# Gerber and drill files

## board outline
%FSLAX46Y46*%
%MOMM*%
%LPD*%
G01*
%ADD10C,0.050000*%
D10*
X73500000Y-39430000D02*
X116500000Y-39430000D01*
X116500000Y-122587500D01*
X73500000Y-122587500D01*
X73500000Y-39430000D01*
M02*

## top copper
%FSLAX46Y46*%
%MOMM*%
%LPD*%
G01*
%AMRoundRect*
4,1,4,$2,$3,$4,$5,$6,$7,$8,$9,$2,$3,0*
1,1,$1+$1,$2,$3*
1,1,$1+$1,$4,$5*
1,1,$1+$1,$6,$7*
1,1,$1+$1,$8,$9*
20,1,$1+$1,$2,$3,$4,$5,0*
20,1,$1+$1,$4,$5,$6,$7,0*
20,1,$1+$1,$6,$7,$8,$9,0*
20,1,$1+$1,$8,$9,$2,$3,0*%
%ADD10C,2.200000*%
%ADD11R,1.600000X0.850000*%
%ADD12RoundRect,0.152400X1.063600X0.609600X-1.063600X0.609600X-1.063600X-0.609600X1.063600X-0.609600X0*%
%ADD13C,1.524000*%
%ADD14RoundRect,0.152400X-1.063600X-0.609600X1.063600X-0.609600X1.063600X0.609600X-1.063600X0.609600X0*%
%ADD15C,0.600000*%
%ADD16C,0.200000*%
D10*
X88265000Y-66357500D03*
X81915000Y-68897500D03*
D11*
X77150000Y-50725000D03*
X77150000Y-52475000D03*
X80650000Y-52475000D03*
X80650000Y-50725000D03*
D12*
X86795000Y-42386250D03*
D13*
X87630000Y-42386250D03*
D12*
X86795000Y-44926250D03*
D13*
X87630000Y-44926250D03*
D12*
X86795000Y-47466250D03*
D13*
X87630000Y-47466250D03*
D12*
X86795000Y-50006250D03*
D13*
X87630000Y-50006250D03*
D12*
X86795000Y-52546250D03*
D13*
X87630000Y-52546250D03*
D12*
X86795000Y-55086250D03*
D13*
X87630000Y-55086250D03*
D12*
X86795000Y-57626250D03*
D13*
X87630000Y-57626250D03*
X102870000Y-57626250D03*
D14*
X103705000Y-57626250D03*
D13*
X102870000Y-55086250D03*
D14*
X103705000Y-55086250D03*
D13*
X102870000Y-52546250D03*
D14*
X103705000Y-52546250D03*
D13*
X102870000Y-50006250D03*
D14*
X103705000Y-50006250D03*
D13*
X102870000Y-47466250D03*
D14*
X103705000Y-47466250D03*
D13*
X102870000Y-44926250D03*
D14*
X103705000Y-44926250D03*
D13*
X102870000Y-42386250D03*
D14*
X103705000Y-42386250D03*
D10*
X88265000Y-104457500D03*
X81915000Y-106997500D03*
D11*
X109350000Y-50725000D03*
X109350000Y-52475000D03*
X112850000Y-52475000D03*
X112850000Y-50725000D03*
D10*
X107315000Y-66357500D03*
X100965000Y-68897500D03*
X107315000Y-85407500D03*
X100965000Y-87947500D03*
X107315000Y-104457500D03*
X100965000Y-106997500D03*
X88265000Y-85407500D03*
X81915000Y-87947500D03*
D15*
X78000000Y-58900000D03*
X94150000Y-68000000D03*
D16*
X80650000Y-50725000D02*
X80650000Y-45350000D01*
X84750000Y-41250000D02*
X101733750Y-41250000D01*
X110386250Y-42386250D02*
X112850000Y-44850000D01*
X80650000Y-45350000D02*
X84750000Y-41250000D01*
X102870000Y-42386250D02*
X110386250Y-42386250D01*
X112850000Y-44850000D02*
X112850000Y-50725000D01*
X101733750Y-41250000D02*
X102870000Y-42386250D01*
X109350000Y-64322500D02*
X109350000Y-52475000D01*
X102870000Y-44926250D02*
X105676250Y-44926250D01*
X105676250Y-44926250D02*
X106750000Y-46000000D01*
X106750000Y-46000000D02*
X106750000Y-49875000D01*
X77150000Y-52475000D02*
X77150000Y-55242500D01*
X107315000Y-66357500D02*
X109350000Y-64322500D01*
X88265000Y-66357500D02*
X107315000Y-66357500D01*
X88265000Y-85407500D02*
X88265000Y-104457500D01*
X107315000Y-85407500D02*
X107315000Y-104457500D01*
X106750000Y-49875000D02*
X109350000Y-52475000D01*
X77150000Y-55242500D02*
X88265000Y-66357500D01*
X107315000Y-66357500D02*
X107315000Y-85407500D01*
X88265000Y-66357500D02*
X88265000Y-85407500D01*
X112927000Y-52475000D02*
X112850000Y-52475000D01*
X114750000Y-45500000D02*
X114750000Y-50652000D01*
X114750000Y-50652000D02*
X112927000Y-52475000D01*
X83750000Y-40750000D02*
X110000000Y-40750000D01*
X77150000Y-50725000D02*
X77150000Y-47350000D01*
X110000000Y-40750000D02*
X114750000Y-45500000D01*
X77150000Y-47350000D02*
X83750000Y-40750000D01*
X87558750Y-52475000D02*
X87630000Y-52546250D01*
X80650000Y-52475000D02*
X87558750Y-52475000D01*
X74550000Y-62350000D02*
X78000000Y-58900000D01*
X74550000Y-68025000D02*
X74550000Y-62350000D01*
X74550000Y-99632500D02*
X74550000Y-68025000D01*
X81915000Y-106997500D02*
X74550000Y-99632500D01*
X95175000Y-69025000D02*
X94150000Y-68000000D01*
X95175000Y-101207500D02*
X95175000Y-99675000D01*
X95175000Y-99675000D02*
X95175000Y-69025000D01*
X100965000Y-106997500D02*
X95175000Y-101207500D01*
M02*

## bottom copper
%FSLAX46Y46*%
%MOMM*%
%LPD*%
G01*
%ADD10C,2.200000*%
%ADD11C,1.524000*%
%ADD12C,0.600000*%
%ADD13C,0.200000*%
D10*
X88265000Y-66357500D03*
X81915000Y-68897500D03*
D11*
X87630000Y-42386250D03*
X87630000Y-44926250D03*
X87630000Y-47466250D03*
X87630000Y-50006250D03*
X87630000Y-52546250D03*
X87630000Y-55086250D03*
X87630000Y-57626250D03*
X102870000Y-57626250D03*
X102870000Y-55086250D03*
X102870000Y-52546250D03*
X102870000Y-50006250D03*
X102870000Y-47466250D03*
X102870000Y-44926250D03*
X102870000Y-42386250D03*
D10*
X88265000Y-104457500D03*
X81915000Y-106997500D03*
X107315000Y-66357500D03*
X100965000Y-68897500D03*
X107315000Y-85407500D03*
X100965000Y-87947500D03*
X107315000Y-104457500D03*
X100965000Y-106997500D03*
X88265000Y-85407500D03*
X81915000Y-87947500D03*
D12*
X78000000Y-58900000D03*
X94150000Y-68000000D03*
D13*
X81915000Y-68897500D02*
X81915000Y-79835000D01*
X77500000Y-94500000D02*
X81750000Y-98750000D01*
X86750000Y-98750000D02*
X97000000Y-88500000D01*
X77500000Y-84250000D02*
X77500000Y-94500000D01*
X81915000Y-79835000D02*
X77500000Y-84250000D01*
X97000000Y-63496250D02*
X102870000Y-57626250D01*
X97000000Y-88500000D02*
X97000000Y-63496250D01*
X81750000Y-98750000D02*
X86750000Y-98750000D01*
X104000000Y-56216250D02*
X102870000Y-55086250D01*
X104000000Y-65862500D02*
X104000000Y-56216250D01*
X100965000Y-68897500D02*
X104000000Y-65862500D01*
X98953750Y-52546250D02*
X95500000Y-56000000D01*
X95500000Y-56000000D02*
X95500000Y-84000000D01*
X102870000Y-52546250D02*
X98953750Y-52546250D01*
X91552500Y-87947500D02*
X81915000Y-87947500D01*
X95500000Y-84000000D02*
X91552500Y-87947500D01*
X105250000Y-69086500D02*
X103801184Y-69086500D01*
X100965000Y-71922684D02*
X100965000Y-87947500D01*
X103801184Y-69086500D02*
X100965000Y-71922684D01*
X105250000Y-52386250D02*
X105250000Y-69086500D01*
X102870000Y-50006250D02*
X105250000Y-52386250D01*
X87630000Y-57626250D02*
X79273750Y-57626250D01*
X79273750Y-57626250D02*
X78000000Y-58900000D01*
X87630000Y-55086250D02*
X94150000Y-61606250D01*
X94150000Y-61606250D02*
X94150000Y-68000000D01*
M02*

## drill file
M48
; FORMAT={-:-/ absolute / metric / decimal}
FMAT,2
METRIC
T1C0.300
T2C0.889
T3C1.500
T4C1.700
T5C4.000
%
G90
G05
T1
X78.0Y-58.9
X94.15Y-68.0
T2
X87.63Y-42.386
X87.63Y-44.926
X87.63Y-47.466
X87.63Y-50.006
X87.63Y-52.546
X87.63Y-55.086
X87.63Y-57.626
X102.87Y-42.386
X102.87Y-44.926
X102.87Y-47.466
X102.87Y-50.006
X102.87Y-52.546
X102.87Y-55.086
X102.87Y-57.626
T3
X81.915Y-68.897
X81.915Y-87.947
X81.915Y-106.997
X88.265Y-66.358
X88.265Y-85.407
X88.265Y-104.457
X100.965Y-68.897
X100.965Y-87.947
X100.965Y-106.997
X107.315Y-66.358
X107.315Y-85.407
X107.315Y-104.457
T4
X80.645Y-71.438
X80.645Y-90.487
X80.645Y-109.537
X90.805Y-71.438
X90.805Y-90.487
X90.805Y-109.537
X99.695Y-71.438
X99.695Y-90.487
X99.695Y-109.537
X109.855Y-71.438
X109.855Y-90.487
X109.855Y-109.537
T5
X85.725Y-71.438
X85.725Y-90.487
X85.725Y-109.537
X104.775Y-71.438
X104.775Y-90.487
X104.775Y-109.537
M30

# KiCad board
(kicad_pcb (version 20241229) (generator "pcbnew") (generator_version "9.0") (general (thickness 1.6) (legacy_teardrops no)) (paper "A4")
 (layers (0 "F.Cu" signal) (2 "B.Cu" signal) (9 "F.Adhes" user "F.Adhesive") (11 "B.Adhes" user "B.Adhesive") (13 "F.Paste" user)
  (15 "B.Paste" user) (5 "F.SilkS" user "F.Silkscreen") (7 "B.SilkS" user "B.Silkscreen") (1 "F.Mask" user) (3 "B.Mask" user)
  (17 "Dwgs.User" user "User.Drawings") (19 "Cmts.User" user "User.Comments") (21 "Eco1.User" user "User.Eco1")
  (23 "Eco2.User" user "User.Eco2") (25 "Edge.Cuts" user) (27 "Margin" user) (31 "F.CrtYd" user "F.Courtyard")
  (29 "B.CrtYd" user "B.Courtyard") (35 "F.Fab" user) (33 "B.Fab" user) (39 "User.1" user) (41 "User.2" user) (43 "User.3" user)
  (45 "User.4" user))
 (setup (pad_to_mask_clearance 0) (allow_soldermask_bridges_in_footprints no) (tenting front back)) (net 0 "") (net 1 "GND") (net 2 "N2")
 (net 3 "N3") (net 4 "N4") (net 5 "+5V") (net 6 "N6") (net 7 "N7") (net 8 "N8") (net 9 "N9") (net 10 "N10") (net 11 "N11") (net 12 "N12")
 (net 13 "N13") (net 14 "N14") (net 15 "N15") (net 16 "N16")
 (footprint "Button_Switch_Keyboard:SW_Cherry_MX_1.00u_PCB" (layer "F.Cu") (at 88.265 66.3575)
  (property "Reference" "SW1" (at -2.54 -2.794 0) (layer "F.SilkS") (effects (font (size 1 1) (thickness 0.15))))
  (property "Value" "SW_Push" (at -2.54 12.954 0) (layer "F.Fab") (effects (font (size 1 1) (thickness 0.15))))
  (pad "" np_thru_hole circle (at -7.62 5.08) (size 1.7 1.7) (drill 1.7) (layers "*.Cu" "*.Mask"))
  (pad "" np_thru_hole circle (at -2.54 5.08) (size 4 4) (drill 4) (layers "*.Cu" "*.Mask"))
  (pad "" np_thru_hole circle (at 2.54 5.08) (size 1.7 1.7) (drill 1.7) (layers "*.Cu" "*.Mask"))
  (pad "1" thru_hole circle (at 0 0) (size 2.2 2.2) (drill 1.5) (layers "*.Cu" "*.Mask") (remove_unused_layers no) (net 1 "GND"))
  (pad "2" thru_hole circle (at -6.35 2.54) (size 2.2 2.2) (drill 1.5) (layers "*.Cu" "*.Mask") (remove_unused_layers no) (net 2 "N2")))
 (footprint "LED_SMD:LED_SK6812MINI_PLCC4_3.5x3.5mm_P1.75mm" (layer "F.Cu") (at 78.9 51.6)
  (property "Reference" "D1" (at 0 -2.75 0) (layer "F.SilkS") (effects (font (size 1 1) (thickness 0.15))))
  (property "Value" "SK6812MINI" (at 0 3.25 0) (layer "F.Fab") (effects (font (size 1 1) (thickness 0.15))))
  (pad "1" smd rect (at -1.75 -0.875) (size 1.6 0.85) (layers "F.Cu" "F.Mask" "F.Paste") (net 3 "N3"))
  (pad "2" smd rect (at -1.75 0.875) (size 1.6 0.85) (layers "F.Cu" "F.Mask" "F.Paste") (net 1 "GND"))
  (pad "3" smd rect (at 1.75 0.875) (size 1.6 0.85) (layers "F.Cu" "F.Mask" "F.Paste") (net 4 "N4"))
  (pad "4" smd rect (at 1.75 -0.875) (size 1.6 0.85) (layers "F.Cu" "F.Mask" "F.Paste") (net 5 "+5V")))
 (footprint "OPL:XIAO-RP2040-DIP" (layer "F.Cu") (at 95.25 50.00625)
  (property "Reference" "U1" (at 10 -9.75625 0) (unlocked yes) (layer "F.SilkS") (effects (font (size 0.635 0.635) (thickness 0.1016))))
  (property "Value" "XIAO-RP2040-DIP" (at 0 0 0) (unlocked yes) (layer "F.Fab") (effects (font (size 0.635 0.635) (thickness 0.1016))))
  (pad "1" smd roundrect (at -8.455 -7.62 180) (size 2.432 1.524) (layers "F.Cu" "F.Mask") (roundrect_rratio 0.1) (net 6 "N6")
   (thermal_bridge_angle 45))
  (pad "1" thru_hole circle (at -7.62 -7.62 180) (size 1.524 1.524) (drill 0.889) (layers "*.Cu" "*.Mask") (remove_unused_layers no)
   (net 6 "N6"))
  (pad "2" smd roundrect (at -8.455 -5.08 180) (size 2.432 1.524) (layers "F.Cu" "F.Mask") (roundrect_rratio 0.1) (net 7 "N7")
   (thermal_bridge_angle 45))
  (pad "2" thru_hole circle (at -7.62 -5.08 180) (size 1.524 1.524) (drill 0.889) (layers "*.Cu" "*.Mask") (remove_unused_layers no)
   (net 7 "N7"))
  (pad "3" smd roundrect (at -8.455 -2.54 180) (size 2.432 1.524) (layers "F.Cu" "F.Mask") (roundrect_rratio 0.1) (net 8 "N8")
   (thermal_bridge_angle 45))
  (pad "3" thru_hole circle (at -7.62 -2.54 180) (size 1.524 1.524) (drill 0.889) (layers "*.Cu" "*.Mask") (remove_unused_layers no)
   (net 8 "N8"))
  (pad "4" smd roundrect (at -8.455 0 180) (size 2.432 1.524) (layers "F.Cu" "F.Mask") (roundrect_rratio 0.1) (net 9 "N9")
   (thermal_bridge_angle 45))
  (pad "4" thru_hole circle (at -7.62 0 180) (size 1.524 1.524) (drill 0.889) (layers "*.Cu" "*.Mask") (remove_unused_layers no)
   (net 9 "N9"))
  (pad "5" smd roundrect (at -8.455 2.54 180) (size 2.432 1.524) (layers "F.Cu" "F.Mask") (roundrect_rratio 0.1) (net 4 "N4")
   (thermal_bridge_angle 45))
  (pad "5" thru_hole circle (at -7.62 2.54 180) (size 1.524 1.524) (drill 0.889) (layers "*.Cu" "*.Mask") (remove_unused_layers no)
   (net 4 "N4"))
  (pad "6" smd roundrect (at -8.455 5.08 180) (size 2.432 1.524) (layers "F.Cu" "F.Mask") (roundrect_rratio 0.1) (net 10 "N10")
   (thermal_bridge_angle 45))
  (pad "6" thru_hole circle (at -7.62 5.08 180) (size 1.524 1.524) (drill 0.889) (layers "*.Cu" "*.Mask") (remove_unused_layers no)
   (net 10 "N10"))
  (pad "7" smd roundrect (at -8.455 7.62 180) (size 2.432 1.524) (layers "F.Cu" "F.Mask") (roundrect_rratio 0.1) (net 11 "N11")
   (thermal_bridge_angle 45))
  (pad "7" thru_hole circle (at -7.62 7.62 180) (size 1.524 1.524) (drill 0.889) (layers "*.Cu" "*.Mask") (remove_unused_layers no)
   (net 11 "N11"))
  (pad "8" thru_hole circle (at 7.62 7.62) (size 1.524 1.524) (drill 0.889) (layers "*.Cu" "*.Mask") (remove_unused_layers no) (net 2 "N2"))
  (pad "8" smd roundrect (at 8.455 7.62) (size 2.432 1.524) (layers "F.Cu" "F.Mask") (roundrect_rratio 0.1) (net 2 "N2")
   (thermal_bridge_angle 45))
  (pad "9" thru_hole circle (at 7.62 5.08) (size 1.524 1.524) (drill 0.889) (layers "*.Cu" "*.Mask") (remove_unused_layers no)
   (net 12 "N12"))
  (pad "9" smd roundrect (at 8.455 5.08) (size 2.432 1.524) (layers "F.Cu" "F.Mask") (roundrect_rratio 0.1) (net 12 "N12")
   (thermal_bridge_angle 45))
  (pad "10" thru_hole circle (at 7.62 2.54) (size 1.524 1.524) (drill 0.889) (layers "*.Cu" "*.Mask") (remove_unused_layers no)
   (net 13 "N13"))
  (pad "10" smd roundrect (at 8.455 2.54) (size 2.432 1.524) (layers "F.Cu" "F.Mask") (roundrect_rratio 0.1) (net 13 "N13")
   (thermal_bridge_angle 45))
  (pad "11" thru_hole circle (at 7.62 0) (size 1.524 1.524) (drill 0.889) (layers "*.Cu" "*.Mask") (remove_unused_layers no) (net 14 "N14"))
  (pad "11" smd roundrect (at 8.455 0) (size 2.432 1.524) (layers "F.Cu" "F.Mask") (roundrect_rratio 0.1) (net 14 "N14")
   (thermal_bridge_angle 45))
  (pad "12" thru_hole circle (at 7.62 -2.54) (size 1.524 1.524) (drill 0.889) (layers "*.Cu" "*.Mask") (remove_unused_layers no)
   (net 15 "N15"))
  (pad "12" smd roundrect (at 8.455 -2.54) (size 2.432 1.524) (layers "F.Cu" "F.Mask") (roundrect_rratio 0.1) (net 15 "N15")
   (thermal_bridge_angle 45))
  (pad "13" thru_hole circle (at 7.62 -5.08) (size 1.524 1.524) (drill 0.889) (layers "*.Cu" "*.Mask") (remove_unused_layers no)
   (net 1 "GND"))
  (pad "13" smd roundrect (at 8.455 -5.08) (size 2.432 1.524) (layers "F.Cu" "F.Mask") (roundrect_rratio 0.1) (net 1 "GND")
   (thermal_bridge_angle 45))
  (pad "14" thru_hole circle (at 7.62 -7.62) (size 1.524 1.524) (drill 0.889) (layers "*.Cu" "*.Mask") (remove_unused_layers no)
   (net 5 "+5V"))
  (pad "14" smd roundrect (at 8.455 -7.62) (size 2.432 1.524) (layers "F.Cu" "F.Mask") (roundrect_rratio 0.1) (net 5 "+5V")
   (thermal_bridge_angle 45)))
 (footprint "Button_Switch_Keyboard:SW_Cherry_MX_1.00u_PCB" (layer "F.Cu") (at 88.265 104.4575)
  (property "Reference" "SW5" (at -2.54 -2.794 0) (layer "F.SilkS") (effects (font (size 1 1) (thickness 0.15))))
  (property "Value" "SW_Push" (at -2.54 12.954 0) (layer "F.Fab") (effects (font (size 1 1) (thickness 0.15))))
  (pad "" np_thru_hole circle (at -7.62 5.08) (size 1.7 1.7) (drill 1.7) (layers "*.Cu" "*.Mask"))
  (pad "" np_thru_hole circle (at -2.54 5.08) (size 4 4) (drill 4) (layers "*.Cu" "*.Mask"))
  (pad "" np_thru_hole circle (at 2.54 5.08) (size 1.7 1.7) (drill 1.7) (layers "*.Cu" "*.Mask"))
  (pad "1" thru_hole circle (at 0 0) (size 2.2 2.2) (drill 1.5) (layers "*.Cu" "*.Mask") (remove_unused_layers no) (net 1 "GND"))
  (pad "2" thru_hole circle (at -6.35 2.54) (size 2.2 2.2) (drill 1.5) (layers "*.Cu" "*.Mask") (remove_unused_layers no) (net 11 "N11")))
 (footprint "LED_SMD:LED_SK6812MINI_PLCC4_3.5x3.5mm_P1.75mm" (layer "F.Cu") (at 111.1 51.6)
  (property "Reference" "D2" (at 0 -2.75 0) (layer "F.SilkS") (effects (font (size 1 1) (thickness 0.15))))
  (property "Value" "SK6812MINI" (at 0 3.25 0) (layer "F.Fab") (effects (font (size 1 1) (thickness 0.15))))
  (pad "1" smd rect (at -1.75 -0.875) (size 1.6 0.85) (layers "F.Cu" "F.Mask" "F.Paste") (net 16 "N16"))
  (pad "2" smd rect (at -1.75 0.875) (size 1.6 0.85) (layers "F.Cu" "F.Mask" "F.Paste") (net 1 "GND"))
  (pad "3" smd rect (at 1.75 0.875) (size 1.6 0.85) (layers "F.Cu" "F.Mask" "F.Paste") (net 3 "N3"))
  (pad "4" smd rect (at 1.75 -0.875) (size 1.6 0.85) (layers "F.Cu" "F.Mask" "F.Paste") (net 5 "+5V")))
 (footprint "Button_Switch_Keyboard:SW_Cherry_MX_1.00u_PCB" (layer "F.Cu") (at 107.315 66.3575)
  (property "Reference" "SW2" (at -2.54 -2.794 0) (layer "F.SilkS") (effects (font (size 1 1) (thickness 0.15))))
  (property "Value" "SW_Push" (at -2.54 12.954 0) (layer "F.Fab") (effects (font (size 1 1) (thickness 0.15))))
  (pad "" np_thru_hole circle (at -7.62 5.08) (size 1.7 1.7) (drill 1.7) (layers "*.Cu" "*.Mask"))
  (pad "" np_thru_hole circle (at -2.54 5.08) (size 4 4) (drill 4) (layers "*.Cu" "*.Mask"))
  (pad "" np_thru_hole circle (at 2.54 5.08) (size 1.7 1.7) (drill 1.7) (layers "*.Cu" "*.Mask"))
  (pad "1" thru_hole circle (at 0 0) (size 2.2 2.2) (drill 1.5) (layers "*.Cu" "*.Mask") (remove_unused_layers no) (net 1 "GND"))
  (pad "2" thru_hole circle (at -6.35 2.54) (size 2.2 2.2) (drill 1.5) (layers "*.Cu" "*.Mask") (remove_unused_layers no) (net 12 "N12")))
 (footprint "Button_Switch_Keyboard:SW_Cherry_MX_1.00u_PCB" (layer "F.Cu") (at 107.315 85.4075)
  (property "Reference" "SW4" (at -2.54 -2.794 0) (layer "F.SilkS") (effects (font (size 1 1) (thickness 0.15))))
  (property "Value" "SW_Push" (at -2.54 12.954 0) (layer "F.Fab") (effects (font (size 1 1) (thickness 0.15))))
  (pad "" np_thru_hole circle (at -7.62 5.08) (size 1.7 1.7) (drill 1.7) (layers "*.Cu" "*.Mask"))
  (pad "" np_thru_hole circle (at -2.54 5.08) (size 4 4) (drill 4) (layers "*.Cu" "*.Mask"))
  (pad "" np_thru_hole circle (at 2.54 5.08) (size 1.7 1.7) (drill 1.7) (layers "*.Cu" "*.Mask"))
  (pad "1" thru_hole circle (at 0 0) (size 2.2 2.2) (drill 1.5) (layers "*.Cu" "*.Mask") (remove_unused_layers no) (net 1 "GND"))
  (pad "2" thru_hole circle (at -6.35 2.54) (size 2.2 2.2) (drill 1.5) (layers "*.Cu" "*.Mask") (remove_unused_layers no) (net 14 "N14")))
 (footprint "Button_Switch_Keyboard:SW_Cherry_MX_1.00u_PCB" (layer "F.Cu") (at 107.315 104.4575)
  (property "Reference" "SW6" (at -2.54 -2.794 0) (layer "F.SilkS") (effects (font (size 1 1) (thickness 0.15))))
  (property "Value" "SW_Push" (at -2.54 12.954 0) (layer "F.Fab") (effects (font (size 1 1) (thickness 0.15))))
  (pad "" np_thru_hole circle (at -7.62 5.08) (size 1.7 1.7) (drill 1.7) (layers "*.Cu" "*.Mask"))
  (pad "" np_thru_hole circle (at -2.54 5.08) (size 4 4) (drill 4) (layers "*.Cu" "*.Mask"))
  (pad "" np_thru_hole circle (at 2.54 5.08) (size 1.7 1.7) (drill 1.7) (layers "*.Cu" "*.Mask"))
  (pad "1" thru_hole circle (at 0 0) (size 2.2 2.2) (drill 1.5) (layers "*.Cu" "*.Mask") (remove_unused_layers no) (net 1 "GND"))
  (pad "2" thru_hole circle (at -6.35 2.54) (size 2.2 2.2) (drill 1.5) (layers "*.Cu" "*.Mask") (remove_unused_layers no) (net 10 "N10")))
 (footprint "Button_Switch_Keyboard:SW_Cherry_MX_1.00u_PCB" (layer "F.Cu") (at 88.265 85.4075)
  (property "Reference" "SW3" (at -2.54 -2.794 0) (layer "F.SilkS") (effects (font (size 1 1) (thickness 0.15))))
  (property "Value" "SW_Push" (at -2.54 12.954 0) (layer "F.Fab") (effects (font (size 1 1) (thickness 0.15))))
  (pad "" np_thru_hole circle (at -7.62 5.08) (size 1.7 1.7) (drill 1.7) (layers "*.Cu" "*.Mask"))
  (pad "" np_thru_hole circle (at -2.54 5.08) (size 4 4) (drill 4) (layers "*.Cu" "*.Mask"))
  (pad "" np_thru_hole circle (at 2.54 5.08) (size 1.7 1.7) (drill 1.7) (layers "*.Cu" "*.Mask"))
  (pad "1" thru_hole circle (at 0 0) (size 2.2 2.2) (drill 1.5) (layers "*.Cu" "*.Mask") (remove_unused_layers no) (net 1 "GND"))
  (pad "2" thru_hole circle (at -6.35 2.54) (size 2.2 2.2) (drill 1.5) (layers "*.Cu" "*.Mask") (remove_unused_layers no) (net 13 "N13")))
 (gr_rect (start 73.5 39.43) (end 116.5 122.5875) (stroke (width 0.05) (type default)) (fill no) (layer "Edge.Cuts"))
 (segment (start 80.65 50.725) (end 80.65 45.35) (width 0.2) (layer "F.Cu") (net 5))
 (segment (start 84.75 41.25) (end 101.73375 41.25) (width 0.2) (layer "F.Cu") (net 5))
 (segment (start 110.38625 42.38625) (end 112.85 44.85) (width 0.2) (layer "F.Cu") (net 5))
 (segment (start 80.65 45.35) (end 84.75 41.25) (width 0.2) (layer "F.Cu") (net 5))
 (segment (start 102.87 42.38625) (end 110.38625 42.38625) (width 0.2) (layer "F.Cu") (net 5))
 (segment (start 112.85 44.85) (end 112.85 50.725) (width 0.2) (layer "F.Cu") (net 5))
 (segment (start 101.73375 41.25) (end 102.87 42.38625) (width 0.2) (layer "F.Cu") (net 5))
 (segment (start 109.35 64.3225) (end 109.35 52.475) (width 0.2) (layer "F.Cu") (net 1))
 (segment (start 102.87 44.92625) (end 105.67625 44.92625) (width 0.2) (layer "F.Cu") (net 1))
 (segment (start 105.67625 44.92625) (end 106.75 46) (width 0.2) (layer "F.Cu") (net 1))
 (segment (start 106.75 46) (end 106.75 49.875) (width 0.2) (layer "F.Cu") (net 1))
 (segment (start 77.15 52.475) (end 77.15 55.2425) (width 0.2) (layer "F.Cu") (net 1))
 (segment (start 107.315 66.3575) (end 109.35 64.3225) (width 0.2) (layer "F.Cu") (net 1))
 (segment (start 88.265 66.3575) (end 107.315 66.3575) (width 0.2) (layer "F.Cu") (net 1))
 (segment (start 88.265 85.4075) (end 88.265 104.4575) (width 0.2) (layer "F.Cu") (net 1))
 (segment (start 107.315 85.4075) (end 107.315 104.4575) (width 0.2) (layer "F.Cu") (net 1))
 (segment (start 106.75 49.875) (end 109.35 52.475) (width 0.2) (layer "F.Cu") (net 1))
 (segment (start 77.15 55.2425) (end 88.265 66.3575) (width 0.2) (layer "F.Cu") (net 1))
 (segment (start 107.315 66.3575) (end 107.315 85.4075) (width 0.2) (layer "F.Cu") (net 1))
 (segment (start 88.265 66.3575) (end 88.265 85.4075) (width 0.2) (layer "F.Cu") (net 1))
 (segment (start 112.927 52.475) (end 112.85 52.475) (width 0.2) (layer "F.Cu") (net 3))
 (segment (start 114.75 45.5) (end 114.75 50.652) (width 0.2) (layer "F.Cu") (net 3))
 (segment (start 114.75 50.652) (end 112.927 52.475) (width 0.2) (layer "F.Cu") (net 3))
 (segment (start 83.75 40.75) (end 110 40.75) (width 0.2) (layer "F.Cu") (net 3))
 (segment (start 77.15 50.725) (end 77.15 47.35) (width 0.2) (layer "F.Cu") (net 3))
 (segment (start 110 40.75) (end 114.75 45.5) (width 0.2) (layer "F.Cu") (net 3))
 (segment (start 77.15 47.35) (end 83.75 40.75) (width 0.2) (layer "F.Cu") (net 3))
 (segment (start 87.55875 52.475) (end 87.63 52.54625) (width 0.2) (layer "F.Cu") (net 4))
 (segment (start 80.65 52.475) (end 87.55875 52.475) (width 0.2) (layer "F.Cu") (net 4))
 (segment (start 81.915 68.8975) (end 81.915 79.835) (width 0.2) (layer "B.Cu") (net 2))
 (segment (start 77.5 94.5) (end 81.75 98.75) (width 0.2) (layer "B.Cu") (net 2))
 (segment (start 86.75 98.75) (end 97 88.5) (width 0.2) (layer "B.Cu") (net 2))
 (segment (start 77.5 84.25) (end 77.5 94.5) (width 0.2) (layer "B.Cu") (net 2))
 (segment (start 81.915 79.835) (end 77.5 84.25) (width 0.2) (layer "B.Cu") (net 2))
 (segment (start 97 63.49625) (end 102.87 57.62625) (width 0.2) (layer "B.Cu") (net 2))
 (segment (start 97 88.5) (end 97 63.49625) (width 0.2) (layer "B.Cu") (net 2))
 (segment (start 81.75 98.75) (end 86.75 98.75) (width 0.2) (layer "B.Cu") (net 2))
 (segment (start 104 56.21625) (end 102.87 55.08625) (width 0.2) (layer "B.Cu") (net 12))
 (segment (start 104 65.8625) (end 104 56.21625) (width 0.2) (layer "B.Cu") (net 12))
 (segment (start 100.965 68.8975) (end 104 65.8625) (width 0.2) (layer "B.Cu") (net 12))
 (segment (start 98.95375 52.54625) (end 95.5 56) (width 0.2) (layer "B.Cu") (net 13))
 (segment (start 95.5 56) (end 95.5 84) (width 0.2) (layer "B.Cu") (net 13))
 (segment (start 102.87 52.54625) (end 98.95375 52.54625) (width 0.2) (layer "B.Cu") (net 13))
 (segment (start 91.5525 87.9475) (end 81.915 87.9475) (width 0.2) (layer "B.Cu") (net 13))
 (segment (start 95.5 84) (end 91.5525 87.9475) (width 0.2) (layer "B.Cu") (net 13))
 (segment (start 105.25 69.0865) (end 103.801184 69.0865) (width 0.2) (layer "B.Cu") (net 14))
 (segment (start 100.965 71.922684) (end 100.965 87.9475) (width 0.2) (layer "B.Cu") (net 14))
 (segment (start 103.801184 69.0865) (end 100.965 71.922684) (width 0.2) (layer "B.Cu") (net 14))
 (segment (start 105.25 52.38625) (end 105.25 69.0865) (width 0.2) (layer "B.Cu") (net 14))
 (segment (start 102.87 50.00625) (end 105.25 52.38625) (width 0.2) (layer "B.Cu") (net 14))
 (segment (start 74.55 62.35) (end 78 58.9) (width 0.2) (layer "F.Cu") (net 11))
 (segment (start 74.55 68.025) (end 74.55 62.35) (width 0.2) (layer "F.Cu") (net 11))
 (segment (start 74.55 99.6325) (end 74.55 68.025) (width 0.2) (layer "F.Cu") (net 11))
 (segment (start 81.915 106.9975) (end 74.55 99.6325) (width 0.2) (layer "F.Cu") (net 11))
 (via (at 78 58.9) (size 0.6) (drill 0.3) (layers "F.Cu" "B.Cu") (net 11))
 (segment (start 87.63 57.62625) (end 79.27375 57.62625) (width 0.2) (layer "B.Cu") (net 11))
 (segment (start 79.27375 57.62625) (end 78 58.9) (width 0.2) (layer "B.Cu") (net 11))
 (segment (start 95.175 69.025) (end 94.15 68) (width 0.2) (layer "F.Cu") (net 10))
 (segment (start 95.175 101.2075) (end 95.175 99.675) (width 0.2) (layer "F.Cu") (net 10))
 (segment (start 95.175 99.675) (end 95.175 69.025) (width 0.2) (layer "F.Cu") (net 10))
 (segment (start 100.965 106.9975) (end 95.175 101.2075) (width 0.2) (layer "F.Cu") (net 10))
 (via (at 94.15 68) (size 0.6) (drill 0.3) (layers "F.Cu" "B.Cu") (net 10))
 (segment (start 87.63 55.08625) (end 94.15 61.60625) (width 0.2) (layer "B.Cu") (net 10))
 (segment (start 94.15 61.60625) (end 94.15 68) (width 0.2) (layer "B.Cu") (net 10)))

